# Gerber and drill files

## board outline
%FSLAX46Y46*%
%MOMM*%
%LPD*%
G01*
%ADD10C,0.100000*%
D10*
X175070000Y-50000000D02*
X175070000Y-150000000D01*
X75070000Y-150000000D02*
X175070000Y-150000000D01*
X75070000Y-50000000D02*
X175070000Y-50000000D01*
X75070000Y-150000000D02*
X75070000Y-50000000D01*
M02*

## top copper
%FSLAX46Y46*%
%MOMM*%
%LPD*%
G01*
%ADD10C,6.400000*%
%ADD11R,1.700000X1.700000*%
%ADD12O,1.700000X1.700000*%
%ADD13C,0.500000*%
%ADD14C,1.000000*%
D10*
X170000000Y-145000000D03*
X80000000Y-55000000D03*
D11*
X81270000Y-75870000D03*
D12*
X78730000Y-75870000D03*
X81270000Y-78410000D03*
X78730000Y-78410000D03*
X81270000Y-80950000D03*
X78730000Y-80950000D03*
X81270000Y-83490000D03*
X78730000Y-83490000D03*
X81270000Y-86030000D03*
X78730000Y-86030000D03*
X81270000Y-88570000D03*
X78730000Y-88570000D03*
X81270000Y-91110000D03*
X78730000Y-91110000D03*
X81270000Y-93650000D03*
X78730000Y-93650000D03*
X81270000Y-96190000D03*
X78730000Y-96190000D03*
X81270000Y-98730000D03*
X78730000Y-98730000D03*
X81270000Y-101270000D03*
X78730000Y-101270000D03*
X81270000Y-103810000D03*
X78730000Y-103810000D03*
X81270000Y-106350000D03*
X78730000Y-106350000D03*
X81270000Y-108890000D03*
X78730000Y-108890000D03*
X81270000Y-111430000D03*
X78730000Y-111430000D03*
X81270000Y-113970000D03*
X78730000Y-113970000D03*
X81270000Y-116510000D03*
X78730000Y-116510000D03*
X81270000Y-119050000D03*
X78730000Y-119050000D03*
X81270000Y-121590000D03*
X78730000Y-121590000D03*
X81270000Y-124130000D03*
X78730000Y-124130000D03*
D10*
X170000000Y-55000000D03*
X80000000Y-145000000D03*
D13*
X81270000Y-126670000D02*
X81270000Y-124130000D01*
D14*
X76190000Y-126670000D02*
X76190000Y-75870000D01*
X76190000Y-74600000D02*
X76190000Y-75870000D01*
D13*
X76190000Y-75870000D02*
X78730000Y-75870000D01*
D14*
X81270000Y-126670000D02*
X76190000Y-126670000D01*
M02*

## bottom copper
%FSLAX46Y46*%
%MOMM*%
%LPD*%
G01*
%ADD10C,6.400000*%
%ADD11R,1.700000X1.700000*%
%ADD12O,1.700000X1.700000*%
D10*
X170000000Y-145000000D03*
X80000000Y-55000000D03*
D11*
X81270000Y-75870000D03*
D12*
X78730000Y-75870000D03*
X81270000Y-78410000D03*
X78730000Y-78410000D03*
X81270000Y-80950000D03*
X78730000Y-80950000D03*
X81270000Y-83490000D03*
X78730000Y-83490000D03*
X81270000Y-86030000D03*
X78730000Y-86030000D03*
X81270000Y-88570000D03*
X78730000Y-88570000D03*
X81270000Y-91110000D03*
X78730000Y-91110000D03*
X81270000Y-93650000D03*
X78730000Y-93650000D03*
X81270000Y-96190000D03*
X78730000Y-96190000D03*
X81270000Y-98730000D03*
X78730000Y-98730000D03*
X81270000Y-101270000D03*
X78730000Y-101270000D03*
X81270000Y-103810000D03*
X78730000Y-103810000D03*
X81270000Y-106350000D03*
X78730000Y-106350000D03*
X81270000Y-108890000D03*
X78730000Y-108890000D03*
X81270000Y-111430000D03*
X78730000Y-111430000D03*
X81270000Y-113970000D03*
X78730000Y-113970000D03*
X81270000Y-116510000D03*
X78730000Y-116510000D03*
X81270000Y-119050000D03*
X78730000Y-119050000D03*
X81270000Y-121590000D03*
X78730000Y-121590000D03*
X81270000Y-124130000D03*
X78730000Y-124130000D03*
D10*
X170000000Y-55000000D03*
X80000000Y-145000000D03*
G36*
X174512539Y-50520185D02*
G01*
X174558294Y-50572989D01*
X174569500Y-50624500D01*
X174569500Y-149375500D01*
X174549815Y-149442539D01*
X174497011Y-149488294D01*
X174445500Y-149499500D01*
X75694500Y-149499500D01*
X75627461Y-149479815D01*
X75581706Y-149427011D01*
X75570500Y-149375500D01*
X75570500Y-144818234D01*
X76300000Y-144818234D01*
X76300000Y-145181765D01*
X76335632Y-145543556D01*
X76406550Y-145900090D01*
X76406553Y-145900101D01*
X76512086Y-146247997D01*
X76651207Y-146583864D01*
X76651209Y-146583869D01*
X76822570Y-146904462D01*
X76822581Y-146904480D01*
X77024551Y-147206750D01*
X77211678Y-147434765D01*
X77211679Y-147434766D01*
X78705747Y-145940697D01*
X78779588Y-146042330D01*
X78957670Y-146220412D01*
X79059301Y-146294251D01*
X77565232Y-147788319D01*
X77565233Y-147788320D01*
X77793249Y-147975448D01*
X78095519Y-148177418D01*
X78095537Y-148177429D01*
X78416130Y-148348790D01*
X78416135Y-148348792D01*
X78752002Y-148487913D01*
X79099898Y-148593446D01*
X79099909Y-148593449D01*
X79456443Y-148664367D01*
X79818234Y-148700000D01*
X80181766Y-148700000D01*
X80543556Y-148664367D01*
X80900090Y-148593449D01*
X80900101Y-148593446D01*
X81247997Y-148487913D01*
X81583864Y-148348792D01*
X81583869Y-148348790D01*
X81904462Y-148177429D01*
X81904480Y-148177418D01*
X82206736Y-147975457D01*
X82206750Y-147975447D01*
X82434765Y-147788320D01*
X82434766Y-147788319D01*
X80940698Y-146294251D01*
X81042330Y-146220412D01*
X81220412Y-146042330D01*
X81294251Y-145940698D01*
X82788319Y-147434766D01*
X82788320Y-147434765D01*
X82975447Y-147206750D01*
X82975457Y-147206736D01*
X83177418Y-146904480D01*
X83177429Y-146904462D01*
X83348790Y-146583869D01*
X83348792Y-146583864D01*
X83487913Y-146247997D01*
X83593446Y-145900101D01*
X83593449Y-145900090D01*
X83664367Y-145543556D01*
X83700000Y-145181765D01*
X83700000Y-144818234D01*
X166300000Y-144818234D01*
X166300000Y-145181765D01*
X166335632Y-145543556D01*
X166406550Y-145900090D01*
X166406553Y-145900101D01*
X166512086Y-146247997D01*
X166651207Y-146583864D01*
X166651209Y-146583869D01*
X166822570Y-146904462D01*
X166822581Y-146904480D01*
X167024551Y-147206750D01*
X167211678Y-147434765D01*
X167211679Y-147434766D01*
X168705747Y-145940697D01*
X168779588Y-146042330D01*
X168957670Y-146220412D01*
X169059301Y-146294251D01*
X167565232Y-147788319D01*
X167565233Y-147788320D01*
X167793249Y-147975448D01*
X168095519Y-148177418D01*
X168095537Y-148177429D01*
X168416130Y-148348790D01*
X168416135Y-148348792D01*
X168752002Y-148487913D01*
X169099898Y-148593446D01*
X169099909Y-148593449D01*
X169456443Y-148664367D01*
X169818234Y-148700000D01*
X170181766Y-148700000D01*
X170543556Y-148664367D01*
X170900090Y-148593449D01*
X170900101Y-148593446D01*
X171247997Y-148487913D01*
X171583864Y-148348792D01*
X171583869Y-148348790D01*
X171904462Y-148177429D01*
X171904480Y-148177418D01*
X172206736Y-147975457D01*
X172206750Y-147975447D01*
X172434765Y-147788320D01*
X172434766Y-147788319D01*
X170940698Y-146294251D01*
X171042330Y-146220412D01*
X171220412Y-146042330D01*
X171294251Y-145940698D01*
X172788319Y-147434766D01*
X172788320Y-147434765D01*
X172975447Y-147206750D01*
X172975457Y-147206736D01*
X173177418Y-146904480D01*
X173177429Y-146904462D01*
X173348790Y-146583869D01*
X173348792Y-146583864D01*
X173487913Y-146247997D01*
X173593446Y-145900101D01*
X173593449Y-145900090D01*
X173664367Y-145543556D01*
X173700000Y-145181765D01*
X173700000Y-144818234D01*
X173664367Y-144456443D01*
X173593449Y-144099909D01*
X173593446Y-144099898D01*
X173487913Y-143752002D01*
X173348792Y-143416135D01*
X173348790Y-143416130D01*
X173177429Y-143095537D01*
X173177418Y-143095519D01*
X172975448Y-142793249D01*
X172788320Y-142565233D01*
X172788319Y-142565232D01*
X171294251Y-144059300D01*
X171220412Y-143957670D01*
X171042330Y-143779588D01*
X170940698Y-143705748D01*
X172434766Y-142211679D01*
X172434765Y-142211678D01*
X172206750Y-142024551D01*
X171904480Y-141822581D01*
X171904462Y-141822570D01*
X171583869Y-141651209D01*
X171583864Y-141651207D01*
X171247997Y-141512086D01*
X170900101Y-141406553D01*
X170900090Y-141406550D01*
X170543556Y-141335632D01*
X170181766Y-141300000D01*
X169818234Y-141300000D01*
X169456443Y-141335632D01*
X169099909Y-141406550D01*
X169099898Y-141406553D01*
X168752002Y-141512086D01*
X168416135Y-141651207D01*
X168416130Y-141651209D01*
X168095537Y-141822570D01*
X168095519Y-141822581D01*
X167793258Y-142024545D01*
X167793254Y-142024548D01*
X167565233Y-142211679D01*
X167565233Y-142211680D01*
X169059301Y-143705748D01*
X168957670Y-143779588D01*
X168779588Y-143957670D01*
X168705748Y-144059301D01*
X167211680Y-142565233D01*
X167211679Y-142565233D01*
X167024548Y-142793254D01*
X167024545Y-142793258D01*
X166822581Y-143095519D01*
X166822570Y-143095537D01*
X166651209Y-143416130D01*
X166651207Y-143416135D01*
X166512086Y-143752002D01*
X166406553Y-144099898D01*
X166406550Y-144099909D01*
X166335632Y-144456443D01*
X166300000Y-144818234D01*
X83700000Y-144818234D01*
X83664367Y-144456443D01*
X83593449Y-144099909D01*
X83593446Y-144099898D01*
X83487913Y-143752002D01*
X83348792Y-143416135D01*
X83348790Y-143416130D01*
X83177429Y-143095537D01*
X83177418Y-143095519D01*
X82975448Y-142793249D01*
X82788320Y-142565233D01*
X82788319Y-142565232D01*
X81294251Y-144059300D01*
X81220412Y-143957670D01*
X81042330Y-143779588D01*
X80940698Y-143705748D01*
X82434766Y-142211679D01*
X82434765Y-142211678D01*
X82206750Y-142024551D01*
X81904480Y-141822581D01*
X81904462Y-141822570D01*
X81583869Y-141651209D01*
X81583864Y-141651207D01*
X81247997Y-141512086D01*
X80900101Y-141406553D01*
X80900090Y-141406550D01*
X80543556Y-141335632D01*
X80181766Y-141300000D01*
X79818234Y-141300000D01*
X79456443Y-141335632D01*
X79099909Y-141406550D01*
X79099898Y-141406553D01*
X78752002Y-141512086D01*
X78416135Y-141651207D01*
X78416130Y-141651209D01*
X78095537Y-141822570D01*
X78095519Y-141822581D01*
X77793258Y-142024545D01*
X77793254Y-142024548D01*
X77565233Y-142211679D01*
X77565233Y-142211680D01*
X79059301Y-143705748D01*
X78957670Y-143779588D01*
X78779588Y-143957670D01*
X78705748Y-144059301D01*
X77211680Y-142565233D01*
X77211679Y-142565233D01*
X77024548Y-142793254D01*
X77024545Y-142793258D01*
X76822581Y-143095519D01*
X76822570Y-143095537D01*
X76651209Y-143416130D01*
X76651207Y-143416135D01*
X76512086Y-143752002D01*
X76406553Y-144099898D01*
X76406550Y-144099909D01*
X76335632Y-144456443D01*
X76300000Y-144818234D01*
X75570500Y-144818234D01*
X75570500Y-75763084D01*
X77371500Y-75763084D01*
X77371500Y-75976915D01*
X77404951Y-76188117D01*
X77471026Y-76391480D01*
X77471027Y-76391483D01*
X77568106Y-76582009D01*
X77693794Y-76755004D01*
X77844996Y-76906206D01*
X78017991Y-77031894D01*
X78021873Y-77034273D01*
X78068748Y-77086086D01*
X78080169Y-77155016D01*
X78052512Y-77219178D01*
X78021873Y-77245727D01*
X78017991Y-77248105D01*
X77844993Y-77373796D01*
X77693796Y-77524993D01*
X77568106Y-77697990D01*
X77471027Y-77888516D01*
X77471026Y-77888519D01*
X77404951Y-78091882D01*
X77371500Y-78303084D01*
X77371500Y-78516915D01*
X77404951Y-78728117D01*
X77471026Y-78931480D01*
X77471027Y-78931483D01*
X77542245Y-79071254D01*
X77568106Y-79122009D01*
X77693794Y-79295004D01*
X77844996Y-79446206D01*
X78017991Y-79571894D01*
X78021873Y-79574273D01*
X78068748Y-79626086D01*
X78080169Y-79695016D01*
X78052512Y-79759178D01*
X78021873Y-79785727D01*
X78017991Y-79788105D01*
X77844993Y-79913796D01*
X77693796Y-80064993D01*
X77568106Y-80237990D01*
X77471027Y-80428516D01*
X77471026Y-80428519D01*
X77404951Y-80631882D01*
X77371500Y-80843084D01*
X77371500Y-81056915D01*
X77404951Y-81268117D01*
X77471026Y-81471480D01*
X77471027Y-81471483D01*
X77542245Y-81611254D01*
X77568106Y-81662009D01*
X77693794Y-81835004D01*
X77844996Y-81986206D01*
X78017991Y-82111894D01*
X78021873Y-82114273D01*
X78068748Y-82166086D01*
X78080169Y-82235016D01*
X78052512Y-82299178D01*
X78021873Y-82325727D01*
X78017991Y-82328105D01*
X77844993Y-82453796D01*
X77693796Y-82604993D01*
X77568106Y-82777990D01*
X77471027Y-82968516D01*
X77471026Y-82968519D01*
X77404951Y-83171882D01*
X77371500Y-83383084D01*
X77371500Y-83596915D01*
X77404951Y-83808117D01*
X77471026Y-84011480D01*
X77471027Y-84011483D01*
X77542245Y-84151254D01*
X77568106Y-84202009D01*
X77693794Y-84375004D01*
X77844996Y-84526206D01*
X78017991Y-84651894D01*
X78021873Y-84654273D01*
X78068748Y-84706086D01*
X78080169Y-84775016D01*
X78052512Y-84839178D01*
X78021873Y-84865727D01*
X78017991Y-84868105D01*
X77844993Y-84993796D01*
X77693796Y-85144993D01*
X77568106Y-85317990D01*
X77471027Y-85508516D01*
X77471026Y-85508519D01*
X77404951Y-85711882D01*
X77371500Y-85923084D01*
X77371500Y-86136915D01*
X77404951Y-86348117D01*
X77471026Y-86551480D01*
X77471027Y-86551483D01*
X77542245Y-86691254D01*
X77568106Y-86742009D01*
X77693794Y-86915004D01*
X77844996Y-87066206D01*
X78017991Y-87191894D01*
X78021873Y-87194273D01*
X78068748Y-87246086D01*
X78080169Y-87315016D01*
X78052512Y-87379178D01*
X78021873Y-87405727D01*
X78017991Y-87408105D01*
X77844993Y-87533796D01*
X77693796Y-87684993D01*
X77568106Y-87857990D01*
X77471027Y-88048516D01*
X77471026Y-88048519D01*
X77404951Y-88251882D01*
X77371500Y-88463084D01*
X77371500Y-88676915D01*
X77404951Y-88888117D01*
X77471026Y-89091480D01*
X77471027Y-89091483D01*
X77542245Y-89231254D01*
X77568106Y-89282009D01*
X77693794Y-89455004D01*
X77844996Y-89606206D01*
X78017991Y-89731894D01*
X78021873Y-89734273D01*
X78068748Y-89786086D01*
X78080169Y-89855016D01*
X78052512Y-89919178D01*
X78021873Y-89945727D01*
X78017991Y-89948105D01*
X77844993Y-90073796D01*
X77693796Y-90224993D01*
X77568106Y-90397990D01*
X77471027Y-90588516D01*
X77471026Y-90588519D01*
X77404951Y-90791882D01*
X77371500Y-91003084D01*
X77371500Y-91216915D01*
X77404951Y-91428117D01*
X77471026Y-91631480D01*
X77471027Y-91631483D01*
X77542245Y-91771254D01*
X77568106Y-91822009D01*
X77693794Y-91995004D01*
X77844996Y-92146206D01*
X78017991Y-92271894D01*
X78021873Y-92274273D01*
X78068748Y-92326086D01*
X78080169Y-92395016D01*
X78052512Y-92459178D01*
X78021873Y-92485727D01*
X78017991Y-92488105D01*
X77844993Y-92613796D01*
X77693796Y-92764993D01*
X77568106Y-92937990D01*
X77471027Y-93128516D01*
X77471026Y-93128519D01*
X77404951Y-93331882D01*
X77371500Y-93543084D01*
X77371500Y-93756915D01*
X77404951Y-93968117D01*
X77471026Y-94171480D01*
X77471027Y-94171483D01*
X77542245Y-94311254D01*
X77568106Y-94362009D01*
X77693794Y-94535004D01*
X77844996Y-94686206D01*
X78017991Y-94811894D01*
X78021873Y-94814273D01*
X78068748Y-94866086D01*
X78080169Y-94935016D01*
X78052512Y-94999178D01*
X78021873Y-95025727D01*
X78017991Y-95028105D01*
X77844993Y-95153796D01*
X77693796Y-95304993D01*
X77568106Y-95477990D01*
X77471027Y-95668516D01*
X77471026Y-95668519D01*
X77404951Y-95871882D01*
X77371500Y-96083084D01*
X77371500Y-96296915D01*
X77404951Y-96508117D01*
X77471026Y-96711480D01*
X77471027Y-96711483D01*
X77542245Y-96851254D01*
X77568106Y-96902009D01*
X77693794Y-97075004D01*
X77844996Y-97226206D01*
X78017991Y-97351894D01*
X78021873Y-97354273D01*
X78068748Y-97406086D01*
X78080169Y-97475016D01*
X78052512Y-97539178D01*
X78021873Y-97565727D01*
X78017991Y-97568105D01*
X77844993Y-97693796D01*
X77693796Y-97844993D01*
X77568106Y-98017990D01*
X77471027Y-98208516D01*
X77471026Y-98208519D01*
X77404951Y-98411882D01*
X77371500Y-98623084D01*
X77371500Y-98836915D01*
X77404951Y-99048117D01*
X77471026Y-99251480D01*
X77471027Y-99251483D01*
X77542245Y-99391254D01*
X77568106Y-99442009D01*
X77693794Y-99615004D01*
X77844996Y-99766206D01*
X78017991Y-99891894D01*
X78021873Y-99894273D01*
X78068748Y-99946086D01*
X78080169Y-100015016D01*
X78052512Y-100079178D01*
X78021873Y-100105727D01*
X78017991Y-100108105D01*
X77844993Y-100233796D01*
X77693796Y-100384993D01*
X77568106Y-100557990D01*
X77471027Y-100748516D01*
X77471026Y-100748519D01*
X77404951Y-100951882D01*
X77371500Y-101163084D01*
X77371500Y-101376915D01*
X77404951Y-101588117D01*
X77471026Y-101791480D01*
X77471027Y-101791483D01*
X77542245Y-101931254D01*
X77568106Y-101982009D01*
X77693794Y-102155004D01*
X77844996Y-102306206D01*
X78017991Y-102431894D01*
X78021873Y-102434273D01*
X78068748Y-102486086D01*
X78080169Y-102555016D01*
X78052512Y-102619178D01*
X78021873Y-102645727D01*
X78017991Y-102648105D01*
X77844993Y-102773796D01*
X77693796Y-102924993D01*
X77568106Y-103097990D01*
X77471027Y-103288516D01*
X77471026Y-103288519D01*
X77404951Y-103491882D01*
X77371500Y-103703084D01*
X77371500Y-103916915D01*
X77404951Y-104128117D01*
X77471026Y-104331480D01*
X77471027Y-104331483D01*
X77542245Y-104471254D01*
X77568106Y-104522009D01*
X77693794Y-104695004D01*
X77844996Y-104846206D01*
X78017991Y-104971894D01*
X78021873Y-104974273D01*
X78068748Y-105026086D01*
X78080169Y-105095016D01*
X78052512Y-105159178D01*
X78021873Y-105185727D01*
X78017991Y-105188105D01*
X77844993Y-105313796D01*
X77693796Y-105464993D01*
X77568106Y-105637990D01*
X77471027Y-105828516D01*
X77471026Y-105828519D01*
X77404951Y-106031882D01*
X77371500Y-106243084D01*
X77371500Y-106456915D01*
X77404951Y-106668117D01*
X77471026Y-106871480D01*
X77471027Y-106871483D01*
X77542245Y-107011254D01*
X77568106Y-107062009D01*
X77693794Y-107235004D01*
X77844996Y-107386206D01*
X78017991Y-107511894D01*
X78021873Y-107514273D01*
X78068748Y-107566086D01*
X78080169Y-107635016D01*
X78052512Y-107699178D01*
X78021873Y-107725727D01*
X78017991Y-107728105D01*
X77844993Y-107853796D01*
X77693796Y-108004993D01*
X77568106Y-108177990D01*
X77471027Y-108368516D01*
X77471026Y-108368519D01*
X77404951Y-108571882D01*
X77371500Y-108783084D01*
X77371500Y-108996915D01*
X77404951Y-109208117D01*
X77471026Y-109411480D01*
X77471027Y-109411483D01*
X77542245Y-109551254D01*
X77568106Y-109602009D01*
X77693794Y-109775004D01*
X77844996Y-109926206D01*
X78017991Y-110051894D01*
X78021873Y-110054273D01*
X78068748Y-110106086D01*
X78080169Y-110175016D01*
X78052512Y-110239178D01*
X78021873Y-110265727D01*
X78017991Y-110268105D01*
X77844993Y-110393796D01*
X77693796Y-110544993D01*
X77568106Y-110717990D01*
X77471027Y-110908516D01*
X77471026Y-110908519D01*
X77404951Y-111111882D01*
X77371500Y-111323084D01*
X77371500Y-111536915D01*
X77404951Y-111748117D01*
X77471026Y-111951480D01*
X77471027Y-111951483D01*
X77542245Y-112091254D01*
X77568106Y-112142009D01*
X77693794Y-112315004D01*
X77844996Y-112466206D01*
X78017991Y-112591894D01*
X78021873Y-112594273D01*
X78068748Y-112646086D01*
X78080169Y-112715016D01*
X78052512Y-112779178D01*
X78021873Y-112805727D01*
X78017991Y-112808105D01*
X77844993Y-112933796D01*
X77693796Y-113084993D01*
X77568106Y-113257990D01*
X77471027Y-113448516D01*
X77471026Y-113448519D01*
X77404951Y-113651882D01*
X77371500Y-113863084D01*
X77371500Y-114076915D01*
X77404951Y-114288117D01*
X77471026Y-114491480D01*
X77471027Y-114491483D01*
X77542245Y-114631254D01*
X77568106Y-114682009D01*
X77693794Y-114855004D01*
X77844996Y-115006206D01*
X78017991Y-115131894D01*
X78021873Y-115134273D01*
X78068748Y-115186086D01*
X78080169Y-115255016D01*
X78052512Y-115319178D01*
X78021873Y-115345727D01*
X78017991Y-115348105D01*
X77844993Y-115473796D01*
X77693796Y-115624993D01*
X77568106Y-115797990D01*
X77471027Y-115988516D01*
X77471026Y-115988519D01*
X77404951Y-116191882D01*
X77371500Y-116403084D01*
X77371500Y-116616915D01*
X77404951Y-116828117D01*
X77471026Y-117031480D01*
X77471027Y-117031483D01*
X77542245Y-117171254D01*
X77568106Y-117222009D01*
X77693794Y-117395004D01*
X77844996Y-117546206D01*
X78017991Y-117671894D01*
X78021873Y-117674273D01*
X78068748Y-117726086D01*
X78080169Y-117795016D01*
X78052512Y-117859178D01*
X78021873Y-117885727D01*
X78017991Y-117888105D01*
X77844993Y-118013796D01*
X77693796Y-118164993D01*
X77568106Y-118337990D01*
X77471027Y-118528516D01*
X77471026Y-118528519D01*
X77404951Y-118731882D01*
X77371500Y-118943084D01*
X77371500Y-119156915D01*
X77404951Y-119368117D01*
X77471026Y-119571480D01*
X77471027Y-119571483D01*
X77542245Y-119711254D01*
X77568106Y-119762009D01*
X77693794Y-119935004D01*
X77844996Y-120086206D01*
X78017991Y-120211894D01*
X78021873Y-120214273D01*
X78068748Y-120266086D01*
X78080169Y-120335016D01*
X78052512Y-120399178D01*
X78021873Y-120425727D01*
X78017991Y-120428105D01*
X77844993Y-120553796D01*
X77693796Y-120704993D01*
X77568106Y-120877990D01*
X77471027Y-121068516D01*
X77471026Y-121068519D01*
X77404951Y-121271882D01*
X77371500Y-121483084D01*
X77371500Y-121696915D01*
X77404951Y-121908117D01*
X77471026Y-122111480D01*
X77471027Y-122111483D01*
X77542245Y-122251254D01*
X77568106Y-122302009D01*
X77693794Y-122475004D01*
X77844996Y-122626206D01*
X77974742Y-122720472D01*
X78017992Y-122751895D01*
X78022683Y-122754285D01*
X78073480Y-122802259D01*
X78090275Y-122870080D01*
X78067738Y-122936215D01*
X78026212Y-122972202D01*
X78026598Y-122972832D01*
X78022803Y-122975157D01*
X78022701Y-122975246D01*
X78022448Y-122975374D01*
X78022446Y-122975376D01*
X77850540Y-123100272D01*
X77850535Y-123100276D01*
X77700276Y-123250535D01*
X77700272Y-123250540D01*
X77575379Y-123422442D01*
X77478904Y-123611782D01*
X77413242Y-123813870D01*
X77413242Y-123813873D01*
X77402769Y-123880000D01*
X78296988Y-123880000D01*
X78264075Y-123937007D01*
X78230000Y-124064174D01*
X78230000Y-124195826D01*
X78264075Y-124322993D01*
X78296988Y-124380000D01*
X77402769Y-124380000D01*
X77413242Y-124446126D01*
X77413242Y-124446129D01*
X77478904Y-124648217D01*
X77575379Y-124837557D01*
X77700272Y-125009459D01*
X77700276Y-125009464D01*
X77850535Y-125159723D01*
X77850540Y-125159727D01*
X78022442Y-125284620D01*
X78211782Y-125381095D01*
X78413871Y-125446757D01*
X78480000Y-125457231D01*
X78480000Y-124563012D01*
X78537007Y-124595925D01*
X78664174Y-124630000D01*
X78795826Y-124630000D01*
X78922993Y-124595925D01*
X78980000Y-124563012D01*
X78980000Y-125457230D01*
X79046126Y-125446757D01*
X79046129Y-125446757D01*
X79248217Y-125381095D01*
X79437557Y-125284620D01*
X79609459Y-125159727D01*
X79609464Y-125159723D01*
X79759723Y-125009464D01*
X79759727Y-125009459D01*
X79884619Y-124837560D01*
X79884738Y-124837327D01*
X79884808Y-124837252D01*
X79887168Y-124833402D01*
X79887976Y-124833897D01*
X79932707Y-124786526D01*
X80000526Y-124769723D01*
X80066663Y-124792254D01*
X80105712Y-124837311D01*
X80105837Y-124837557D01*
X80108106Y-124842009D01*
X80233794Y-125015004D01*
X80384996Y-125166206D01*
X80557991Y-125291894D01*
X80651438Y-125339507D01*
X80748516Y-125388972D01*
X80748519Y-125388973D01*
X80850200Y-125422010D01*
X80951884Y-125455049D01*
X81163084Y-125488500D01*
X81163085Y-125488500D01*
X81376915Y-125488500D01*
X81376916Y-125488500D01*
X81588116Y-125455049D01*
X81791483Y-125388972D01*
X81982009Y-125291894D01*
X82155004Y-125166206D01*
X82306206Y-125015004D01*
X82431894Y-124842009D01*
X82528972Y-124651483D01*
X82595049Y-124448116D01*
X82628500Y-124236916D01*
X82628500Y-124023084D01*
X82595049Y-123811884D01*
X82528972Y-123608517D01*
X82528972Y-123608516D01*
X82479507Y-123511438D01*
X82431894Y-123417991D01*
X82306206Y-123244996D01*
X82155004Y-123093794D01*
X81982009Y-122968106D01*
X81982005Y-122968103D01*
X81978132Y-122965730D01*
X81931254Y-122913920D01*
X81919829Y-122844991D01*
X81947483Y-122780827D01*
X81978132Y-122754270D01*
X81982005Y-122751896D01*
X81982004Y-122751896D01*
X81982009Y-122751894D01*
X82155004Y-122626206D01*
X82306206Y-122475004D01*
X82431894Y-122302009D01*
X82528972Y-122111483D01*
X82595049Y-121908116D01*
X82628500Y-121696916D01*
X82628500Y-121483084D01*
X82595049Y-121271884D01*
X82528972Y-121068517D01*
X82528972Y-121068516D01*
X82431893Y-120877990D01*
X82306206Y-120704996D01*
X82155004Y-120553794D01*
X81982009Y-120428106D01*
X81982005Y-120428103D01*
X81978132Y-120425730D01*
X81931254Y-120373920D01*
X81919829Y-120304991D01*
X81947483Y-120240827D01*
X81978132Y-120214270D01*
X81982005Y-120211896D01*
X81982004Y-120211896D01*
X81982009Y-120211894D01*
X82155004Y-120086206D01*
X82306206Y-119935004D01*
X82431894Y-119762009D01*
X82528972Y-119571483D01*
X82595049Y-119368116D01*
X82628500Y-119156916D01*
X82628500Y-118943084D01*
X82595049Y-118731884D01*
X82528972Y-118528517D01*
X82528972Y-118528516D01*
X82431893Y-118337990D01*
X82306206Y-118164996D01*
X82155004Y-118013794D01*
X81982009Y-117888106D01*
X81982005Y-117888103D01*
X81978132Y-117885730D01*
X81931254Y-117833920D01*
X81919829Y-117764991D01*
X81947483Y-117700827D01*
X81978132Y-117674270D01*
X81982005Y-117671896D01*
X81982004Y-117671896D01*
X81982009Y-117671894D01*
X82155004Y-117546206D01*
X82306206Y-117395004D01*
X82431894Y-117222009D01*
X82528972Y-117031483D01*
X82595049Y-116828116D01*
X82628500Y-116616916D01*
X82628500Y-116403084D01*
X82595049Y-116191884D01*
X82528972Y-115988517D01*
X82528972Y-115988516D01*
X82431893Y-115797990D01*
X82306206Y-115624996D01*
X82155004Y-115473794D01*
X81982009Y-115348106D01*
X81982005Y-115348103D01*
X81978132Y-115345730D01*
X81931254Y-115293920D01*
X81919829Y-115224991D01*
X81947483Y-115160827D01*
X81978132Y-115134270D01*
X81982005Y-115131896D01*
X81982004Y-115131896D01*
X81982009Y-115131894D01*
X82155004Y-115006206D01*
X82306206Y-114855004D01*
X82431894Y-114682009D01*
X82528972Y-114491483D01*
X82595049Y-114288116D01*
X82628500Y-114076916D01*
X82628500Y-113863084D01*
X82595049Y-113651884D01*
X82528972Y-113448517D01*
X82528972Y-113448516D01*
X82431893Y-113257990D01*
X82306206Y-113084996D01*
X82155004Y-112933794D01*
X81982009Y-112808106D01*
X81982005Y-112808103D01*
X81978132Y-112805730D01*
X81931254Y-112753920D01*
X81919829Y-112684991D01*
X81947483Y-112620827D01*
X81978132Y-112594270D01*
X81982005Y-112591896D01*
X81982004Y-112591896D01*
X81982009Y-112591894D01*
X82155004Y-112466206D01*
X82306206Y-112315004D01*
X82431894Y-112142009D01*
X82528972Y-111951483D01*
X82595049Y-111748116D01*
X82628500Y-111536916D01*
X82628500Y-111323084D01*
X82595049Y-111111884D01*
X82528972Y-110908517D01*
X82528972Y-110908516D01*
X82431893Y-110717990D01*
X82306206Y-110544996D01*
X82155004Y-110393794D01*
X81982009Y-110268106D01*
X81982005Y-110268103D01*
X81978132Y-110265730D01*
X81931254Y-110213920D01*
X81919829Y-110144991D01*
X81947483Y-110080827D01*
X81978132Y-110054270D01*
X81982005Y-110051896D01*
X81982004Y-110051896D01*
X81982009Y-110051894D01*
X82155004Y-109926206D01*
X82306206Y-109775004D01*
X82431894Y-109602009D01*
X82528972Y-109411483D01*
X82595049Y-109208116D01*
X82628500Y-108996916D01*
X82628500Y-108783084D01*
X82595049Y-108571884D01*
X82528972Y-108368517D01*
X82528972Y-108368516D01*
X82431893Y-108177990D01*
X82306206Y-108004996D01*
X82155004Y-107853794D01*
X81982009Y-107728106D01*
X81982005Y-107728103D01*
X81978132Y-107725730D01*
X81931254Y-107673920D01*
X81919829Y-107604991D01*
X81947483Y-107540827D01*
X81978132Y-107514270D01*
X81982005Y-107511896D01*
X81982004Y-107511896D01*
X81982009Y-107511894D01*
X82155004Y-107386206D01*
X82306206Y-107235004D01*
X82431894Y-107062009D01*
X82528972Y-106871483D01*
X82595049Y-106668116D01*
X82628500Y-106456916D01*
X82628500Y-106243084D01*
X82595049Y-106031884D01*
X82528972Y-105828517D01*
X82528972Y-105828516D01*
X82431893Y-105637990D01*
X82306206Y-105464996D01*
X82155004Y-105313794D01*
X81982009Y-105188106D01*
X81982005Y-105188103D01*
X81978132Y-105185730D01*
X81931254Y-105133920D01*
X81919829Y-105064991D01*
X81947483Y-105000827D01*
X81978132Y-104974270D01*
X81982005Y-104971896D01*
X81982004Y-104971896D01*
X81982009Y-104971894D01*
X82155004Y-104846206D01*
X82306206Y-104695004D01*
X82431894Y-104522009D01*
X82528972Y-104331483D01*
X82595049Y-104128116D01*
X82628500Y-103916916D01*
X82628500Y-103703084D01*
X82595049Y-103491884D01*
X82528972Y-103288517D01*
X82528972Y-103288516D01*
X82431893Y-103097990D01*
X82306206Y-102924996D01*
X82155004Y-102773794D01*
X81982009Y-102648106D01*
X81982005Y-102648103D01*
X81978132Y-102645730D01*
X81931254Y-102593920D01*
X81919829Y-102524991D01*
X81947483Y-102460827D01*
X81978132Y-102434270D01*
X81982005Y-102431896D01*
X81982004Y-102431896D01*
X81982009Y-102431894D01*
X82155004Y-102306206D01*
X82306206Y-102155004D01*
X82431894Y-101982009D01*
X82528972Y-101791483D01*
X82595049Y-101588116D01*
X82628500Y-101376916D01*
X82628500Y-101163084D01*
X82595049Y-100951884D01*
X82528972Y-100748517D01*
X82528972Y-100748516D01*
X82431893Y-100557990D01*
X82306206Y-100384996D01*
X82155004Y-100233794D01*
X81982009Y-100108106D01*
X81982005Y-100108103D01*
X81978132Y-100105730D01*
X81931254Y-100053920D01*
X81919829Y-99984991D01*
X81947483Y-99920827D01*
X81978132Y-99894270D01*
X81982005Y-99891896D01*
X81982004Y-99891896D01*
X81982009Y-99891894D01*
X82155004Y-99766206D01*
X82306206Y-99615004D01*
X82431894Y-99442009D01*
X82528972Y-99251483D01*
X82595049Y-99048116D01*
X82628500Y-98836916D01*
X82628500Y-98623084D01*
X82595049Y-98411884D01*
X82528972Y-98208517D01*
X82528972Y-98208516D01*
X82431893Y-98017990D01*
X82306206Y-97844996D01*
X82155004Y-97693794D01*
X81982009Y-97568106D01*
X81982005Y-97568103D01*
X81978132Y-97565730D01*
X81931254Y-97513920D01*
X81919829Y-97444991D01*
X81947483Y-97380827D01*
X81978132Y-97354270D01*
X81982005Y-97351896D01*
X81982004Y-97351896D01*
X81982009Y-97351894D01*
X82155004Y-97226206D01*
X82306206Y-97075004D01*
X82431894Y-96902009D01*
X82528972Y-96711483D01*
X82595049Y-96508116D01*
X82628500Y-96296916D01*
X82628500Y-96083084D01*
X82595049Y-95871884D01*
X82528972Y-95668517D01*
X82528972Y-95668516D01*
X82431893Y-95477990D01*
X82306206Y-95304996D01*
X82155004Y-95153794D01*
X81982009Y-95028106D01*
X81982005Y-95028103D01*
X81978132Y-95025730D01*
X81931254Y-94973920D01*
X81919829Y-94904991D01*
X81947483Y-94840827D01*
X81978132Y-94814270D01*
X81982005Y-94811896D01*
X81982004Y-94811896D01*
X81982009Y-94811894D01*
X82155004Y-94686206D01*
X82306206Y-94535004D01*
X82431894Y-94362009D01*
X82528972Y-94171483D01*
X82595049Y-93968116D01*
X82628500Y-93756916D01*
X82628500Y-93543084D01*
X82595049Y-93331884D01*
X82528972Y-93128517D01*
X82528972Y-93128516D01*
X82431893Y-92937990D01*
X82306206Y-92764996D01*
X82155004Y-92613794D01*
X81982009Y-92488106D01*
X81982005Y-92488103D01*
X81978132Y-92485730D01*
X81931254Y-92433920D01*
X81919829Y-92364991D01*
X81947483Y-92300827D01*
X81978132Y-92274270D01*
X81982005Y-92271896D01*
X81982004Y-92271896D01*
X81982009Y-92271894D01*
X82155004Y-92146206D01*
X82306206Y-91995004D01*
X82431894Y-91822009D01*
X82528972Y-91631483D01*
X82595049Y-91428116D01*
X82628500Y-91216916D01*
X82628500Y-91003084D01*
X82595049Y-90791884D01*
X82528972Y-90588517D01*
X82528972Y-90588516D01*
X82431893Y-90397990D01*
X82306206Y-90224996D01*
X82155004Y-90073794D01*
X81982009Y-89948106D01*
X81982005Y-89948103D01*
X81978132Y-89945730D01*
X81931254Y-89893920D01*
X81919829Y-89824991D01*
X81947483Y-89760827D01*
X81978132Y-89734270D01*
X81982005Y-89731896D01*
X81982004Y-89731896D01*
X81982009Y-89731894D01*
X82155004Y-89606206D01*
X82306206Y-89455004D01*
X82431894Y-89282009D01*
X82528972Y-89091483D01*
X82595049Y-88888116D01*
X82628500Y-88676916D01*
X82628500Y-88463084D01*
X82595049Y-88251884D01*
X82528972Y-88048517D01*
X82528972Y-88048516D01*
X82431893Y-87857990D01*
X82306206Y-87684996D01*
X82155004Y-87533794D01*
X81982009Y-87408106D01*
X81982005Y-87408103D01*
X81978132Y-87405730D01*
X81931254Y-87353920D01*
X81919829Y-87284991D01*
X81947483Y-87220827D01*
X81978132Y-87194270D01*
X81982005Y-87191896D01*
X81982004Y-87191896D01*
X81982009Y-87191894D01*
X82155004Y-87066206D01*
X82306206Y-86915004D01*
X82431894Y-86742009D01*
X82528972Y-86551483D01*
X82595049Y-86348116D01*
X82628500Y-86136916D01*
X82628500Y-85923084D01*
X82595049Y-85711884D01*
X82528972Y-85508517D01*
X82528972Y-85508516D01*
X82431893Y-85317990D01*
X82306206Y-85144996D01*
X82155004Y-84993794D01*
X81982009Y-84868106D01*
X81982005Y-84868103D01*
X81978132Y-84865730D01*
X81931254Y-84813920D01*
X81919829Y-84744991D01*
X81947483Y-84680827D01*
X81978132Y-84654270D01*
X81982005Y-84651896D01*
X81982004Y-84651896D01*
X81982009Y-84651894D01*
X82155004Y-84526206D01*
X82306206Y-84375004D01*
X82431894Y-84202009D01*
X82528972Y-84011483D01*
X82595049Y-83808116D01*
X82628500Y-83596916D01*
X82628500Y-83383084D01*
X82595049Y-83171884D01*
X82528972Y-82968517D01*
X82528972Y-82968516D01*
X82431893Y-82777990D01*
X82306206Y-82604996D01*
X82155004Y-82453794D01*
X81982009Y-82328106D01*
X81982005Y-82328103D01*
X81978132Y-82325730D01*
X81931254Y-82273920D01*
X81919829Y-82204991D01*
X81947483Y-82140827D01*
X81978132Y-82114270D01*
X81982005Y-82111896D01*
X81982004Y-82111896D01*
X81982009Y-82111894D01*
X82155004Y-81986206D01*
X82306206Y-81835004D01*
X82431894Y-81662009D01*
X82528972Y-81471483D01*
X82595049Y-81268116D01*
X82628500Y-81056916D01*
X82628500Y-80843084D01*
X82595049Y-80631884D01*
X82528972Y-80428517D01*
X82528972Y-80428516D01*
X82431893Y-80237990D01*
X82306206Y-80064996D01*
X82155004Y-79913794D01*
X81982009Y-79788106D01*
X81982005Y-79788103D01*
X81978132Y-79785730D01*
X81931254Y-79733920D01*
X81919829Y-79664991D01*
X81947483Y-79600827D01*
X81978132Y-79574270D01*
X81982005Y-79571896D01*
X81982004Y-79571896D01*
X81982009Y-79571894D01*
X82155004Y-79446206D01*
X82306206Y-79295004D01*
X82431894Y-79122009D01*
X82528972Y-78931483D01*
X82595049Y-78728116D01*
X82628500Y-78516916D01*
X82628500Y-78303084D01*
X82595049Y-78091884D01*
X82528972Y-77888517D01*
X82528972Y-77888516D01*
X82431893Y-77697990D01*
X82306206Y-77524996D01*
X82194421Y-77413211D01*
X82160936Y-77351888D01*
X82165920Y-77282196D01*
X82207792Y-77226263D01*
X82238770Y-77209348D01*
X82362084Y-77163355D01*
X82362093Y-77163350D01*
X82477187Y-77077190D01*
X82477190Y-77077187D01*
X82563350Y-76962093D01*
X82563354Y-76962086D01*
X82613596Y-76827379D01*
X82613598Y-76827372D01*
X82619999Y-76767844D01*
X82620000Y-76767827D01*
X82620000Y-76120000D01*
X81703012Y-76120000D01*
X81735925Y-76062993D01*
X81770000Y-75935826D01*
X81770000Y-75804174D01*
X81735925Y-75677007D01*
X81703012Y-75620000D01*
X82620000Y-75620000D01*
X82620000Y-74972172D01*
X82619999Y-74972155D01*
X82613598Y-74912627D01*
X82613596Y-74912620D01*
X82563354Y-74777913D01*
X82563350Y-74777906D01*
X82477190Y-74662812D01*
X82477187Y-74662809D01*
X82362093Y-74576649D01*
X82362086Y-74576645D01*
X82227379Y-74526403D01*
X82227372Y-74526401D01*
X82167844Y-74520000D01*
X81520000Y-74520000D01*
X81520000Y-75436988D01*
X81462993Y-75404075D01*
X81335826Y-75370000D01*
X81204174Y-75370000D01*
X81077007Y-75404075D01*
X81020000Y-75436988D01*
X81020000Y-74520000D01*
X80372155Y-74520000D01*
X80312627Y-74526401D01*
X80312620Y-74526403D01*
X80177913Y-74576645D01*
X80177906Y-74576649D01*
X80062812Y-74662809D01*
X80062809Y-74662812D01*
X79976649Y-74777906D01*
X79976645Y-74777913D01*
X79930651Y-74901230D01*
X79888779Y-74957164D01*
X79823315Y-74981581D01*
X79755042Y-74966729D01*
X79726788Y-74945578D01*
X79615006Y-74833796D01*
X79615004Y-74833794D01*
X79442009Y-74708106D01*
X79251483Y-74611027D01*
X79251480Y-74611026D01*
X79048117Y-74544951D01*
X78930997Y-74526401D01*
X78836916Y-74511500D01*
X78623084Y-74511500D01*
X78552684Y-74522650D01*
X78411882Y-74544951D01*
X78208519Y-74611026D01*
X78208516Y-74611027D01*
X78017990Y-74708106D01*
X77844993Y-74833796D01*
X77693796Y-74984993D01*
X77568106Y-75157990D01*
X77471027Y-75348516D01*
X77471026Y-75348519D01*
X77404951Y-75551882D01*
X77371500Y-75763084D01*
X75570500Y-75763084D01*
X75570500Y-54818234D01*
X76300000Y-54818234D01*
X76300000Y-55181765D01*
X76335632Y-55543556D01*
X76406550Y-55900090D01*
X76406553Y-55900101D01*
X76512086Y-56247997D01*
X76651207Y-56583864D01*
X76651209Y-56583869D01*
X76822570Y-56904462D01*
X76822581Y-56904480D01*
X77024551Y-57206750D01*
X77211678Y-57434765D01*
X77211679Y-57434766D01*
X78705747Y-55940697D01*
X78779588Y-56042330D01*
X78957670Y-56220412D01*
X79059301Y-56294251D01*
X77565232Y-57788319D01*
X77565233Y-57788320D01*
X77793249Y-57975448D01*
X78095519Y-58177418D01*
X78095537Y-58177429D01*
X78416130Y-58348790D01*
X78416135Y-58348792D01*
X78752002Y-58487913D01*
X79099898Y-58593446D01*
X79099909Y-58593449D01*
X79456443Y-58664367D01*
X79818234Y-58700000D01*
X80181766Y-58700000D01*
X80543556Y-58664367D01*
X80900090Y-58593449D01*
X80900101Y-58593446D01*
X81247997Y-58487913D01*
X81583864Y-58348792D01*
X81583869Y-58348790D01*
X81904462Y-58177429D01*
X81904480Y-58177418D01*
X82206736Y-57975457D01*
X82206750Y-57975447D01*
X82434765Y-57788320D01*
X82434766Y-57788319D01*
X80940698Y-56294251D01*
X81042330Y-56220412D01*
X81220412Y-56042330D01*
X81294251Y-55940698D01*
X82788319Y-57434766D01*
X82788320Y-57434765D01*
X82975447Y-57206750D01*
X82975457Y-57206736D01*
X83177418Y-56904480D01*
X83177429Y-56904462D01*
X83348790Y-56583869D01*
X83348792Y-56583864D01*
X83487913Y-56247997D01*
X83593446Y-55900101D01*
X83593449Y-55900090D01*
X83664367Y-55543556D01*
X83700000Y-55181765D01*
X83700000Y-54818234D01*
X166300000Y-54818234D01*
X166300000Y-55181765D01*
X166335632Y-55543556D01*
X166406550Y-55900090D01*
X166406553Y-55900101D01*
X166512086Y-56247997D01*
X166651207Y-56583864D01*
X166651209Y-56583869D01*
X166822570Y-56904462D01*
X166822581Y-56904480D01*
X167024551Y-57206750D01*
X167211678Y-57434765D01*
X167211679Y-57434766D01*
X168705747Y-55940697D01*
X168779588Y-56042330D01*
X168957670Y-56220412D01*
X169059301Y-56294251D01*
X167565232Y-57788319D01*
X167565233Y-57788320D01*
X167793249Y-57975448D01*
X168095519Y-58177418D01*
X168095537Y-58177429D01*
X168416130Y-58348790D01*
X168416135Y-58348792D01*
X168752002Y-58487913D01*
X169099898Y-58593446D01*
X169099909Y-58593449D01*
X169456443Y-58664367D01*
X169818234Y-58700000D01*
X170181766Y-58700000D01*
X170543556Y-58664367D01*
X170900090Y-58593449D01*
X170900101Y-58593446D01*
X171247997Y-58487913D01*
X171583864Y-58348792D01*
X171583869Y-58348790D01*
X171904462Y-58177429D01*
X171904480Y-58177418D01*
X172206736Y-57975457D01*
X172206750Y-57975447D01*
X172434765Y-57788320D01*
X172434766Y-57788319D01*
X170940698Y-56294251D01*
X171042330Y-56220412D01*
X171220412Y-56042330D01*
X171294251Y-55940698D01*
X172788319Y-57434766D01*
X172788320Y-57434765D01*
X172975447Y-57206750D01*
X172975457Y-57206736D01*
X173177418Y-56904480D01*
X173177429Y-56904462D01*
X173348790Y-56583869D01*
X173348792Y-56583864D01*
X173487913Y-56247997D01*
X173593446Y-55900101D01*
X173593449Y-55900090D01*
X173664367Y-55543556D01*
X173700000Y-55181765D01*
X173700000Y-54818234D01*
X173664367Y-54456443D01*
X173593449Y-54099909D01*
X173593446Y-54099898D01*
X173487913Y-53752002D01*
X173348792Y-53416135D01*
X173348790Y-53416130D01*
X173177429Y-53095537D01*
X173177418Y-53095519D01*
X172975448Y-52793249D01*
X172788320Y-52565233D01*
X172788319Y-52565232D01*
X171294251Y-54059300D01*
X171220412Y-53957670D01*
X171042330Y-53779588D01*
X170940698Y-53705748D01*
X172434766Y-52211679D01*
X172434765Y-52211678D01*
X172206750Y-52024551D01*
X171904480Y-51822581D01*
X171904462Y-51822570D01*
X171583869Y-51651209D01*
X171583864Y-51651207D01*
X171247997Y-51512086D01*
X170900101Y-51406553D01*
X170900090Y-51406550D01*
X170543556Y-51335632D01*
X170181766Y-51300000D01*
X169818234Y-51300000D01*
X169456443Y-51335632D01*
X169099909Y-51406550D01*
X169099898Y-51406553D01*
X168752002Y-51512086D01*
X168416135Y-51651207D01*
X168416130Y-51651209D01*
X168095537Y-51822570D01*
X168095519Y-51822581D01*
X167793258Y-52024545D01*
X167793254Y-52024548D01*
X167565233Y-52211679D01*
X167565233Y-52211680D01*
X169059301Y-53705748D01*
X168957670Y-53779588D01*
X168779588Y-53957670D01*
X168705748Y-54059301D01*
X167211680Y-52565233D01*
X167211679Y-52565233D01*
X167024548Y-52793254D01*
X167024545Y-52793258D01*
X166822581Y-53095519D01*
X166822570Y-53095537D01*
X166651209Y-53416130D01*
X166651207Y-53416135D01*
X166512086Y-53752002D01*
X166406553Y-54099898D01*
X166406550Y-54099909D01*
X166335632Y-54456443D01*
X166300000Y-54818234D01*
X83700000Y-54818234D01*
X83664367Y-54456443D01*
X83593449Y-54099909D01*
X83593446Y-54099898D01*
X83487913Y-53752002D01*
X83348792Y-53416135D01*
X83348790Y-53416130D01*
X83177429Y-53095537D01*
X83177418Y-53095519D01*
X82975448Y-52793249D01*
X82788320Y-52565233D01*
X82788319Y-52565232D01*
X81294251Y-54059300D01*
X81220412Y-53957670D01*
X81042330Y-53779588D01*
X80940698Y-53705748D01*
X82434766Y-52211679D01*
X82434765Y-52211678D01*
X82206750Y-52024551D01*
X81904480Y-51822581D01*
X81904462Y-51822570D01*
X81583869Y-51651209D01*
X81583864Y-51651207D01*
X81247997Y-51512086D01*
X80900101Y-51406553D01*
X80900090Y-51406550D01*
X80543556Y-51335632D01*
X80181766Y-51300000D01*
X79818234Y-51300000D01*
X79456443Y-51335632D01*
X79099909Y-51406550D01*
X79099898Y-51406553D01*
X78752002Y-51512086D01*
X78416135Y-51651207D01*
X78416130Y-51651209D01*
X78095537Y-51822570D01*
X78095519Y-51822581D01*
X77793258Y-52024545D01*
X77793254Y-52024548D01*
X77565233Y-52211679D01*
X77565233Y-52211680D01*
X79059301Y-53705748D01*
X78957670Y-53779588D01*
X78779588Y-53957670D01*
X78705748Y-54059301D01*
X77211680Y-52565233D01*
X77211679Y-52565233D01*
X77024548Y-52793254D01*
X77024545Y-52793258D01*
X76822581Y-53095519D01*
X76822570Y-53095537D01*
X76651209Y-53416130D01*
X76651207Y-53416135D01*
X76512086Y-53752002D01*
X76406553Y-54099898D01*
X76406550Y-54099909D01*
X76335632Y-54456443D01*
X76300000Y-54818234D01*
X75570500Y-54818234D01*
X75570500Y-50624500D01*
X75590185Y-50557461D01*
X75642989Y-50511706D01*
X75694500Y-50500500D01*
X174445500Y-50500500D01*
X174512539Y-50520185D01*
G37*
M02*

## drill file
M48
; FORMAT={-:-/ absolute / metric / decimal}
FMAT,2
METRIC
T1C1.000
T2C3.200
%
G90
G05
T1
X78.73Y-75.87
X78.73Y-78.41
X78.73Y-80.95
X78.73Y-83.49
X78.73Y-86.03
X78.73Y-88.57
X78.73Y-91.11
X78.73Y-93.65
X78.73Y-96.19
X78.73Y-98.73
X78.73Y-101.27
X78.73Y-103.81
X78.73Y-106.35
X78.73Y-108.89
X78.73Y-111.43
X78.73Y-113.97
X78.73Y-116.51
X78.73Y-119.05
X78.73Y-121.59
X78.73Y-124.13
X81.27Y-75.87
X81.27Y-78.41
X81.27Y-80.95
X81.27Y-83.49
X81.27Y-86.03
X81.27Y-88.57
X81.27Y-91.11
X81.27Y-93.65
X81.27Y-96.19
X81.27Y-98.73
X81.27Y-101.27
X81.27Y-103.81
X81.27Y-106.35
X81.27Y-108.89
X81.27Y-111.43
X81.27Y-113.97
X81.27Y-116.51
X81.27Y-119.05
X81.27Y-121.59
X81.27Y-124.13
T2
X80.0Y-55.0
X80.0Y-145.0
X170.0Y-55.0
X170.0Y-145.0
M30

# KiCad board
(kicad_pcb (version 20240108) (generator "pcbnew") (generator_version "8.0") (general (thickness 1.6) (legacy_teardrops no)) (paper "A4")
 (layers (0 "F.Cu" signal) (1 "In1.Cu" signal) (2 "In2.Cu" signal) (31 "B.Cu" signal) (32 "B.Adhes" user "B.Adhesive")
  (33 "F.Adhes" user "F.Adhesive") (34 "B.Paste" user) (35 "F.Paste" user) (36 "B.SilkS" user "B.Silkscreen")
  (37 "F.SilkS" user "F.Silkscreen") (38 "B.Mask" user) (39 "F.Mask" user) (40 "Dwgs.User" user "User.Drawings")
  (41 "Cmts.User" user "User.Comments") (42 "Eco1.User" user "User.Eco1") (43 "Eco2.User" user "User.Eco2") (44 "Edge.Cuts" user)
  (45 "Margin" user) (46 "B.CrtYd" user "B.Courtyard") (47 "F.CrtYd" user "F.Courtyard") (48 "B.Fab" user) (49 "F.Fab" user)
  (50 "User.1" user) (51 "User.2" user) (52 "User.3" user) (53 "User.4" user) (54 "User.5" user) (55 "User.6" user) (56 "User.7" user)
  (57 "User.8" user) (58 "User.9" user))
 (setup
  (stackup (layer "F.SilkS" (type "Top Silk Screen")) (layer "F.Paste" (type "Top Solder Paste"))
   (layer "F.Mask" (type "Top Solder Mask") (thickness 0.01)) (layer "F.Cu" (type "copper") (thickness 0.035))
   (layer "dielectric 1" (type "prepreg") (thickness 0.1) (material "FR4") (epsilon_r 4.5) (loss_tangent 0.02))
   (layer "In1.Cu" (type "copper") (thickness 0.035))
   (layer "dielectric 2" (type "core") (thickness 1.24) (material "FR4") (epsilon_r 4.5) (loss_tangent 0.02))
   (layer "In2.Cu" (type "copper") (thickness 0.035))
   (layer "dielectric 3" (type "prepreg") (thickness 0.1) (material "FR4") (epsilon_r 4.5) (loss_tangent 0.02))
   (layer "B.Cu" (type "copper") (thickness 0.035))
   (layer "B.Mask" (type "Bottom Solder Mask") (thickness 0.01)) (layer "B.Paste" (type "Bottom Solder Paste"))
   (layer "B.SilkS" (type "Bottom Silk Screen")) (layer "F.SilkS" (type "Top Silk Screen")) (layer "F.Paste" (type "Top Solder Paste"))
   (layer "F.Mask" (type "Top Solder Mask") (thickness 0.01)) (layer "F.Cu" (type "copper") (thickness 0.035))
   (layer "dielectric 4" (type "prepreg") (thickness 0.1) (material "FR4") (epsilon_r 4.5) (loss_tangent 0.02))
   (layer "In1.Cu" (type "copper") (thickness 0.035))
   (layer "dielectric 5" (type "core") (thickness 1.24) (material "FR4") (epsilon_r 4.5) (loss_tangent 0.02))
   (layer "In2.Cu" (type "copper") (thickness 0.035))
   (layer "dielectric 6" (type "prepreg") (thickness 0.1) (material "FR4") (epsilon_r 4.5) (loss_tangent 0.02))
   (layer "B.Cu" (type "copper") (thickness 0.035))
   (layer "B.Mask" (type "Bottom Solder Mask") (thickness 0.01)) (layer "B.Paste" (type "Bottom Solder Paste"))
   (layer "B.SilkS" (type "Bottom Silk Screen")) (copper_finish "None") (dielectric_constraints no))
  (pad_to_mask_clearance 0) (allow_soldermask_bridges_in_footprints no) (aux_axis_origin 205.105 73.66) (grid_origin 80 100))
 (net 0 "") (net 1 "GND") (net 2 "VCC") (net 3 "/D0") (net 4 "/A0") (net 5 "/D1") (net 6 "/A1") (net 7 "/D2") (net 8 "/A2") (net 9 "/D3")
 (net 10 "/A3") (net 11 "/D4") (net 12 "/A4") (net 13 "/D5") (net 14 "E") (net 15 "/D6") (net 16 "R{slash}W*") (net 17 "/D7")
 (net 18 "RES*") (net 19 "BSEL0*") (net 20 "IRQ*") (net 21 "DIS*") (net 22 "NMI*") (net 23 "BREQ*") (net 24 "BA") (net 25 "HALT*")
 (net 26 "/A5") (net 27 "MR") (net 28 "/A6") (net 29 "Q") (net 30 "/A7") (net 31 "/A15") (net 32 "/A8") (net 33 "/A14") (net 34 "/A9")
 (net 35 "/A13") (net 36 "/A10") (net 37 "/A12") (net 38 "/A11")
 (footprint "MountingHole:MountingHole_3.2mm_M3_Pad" (layer "F.Cu") (at 170 145)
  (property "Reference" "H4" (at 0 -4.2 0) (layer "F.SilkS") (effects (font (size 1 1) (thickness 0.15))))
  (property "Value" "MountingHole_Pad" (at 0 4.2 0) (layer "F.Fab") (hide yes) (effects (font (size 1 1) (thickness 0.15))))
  (pad "1" thru_hole circle (at 0 0) (size 6.4 6.4) (drill 3.2) (layers "*.Cu" "*.Mask") (remove_unused_layers no) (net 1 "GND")))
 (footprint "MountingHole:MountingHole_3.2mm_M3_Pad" (layer "F.Cu") (at 80 55)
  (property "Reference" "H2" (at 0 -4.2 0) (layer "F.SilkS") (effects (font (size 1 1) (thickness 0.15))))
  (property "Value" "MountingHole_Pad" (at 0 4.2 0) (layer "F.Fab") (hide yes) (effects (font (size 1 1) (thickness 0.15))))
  (pad "1" thru_hole circle (at 0 0) (size 6.4 6.4) (drill 3.2) (layers "*.Cu" "*.Mask") (remove_unused_layers no) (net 1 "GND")))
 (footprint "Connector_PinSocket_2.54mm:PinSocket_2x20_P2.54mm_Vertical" (layer "F.Cu") (at 81.27 75.87)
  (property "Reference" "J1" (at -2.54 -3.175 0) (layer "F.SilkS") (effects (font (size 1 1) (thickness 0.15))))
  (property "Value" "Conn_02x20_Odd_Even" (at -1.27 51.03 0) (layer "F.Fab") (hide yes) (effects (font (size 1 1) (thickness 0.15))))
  (pad "1" thru_hole rect (at 0 0) (size 1.7 1.7) (drill 1) (layers "*.Cu" "*.Mask") (remove_unused_layers no) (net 1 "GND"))
  (pad "2" thru_hole oval (at -2.54 0) (size 1.7 1.7) (drill 1) (layers "*.Cu" "*.Mask") (remove_unused_layers no) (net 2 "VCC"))
  (pad "3" thru_hole oval (at 0 2.54) (size 1.7 1.7) (drill 1) (layers "*.Cu" "*.Mask") (remove_unused_layers no) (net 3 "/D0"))
  (pad "4" thru_hole oval (at -2.54 2.54) (size 1.7 1.7) (drill 1) (layers "*.Cu" "*.Mask") (remove_unused_layers no) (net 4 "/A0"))
  (pad "5" thru_hole oval (at 0 5.08) (size 1.7 1.7) (drill 1) (layers "*.Cu" "*.Mask") (remove_unused_layers no) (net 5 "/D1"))
  (pad "6" thru_hole oval (at -2.54 5.08) (size 1.7 1.7) (drill 1) (layers "*.Cu" "*.Mask") (remove_unused_layers no) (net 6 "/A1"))
  (pad "7" thru_hole oval (at 0 7.62) (size 1.7 1.7) (drill 1) (layers "*.Cu" "*.Mask") (remove_unused_layers no) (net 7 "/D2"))
  (pad "8" thru_hole oval (at -2.54 7.62) (size 1.7 1.7) (drill 1) (layers "*.Cu" "*.Mask") (remove_unused_layers no) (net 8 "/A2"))
  (pad "9" thru_hole oval (at 0 10.16) (size 1.7 1.7) (drill 1) (layers "*.Cu" "*.Mask") (remove_unused_layers no) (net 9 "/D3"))
  (pad "10" thru_hole oval (at -2.54 10.16) (size 1.7 1.7) (drill 1) (layers "*.Cu" "*.Mask") (remove_unused_layers no) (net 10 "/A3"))
  (pad "11" thru_hole oval (at 0 12.7) (size 1.7 1.7) (drill 1) (layers "*.Cu" "*.Mask") (remove_unused_layers no) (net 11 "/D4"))
  (pad "12" thru_hole oval (at -2.54 12.7) (size 1.7 1.7) (drill 1) (layers "*.Cu" "*.Mask") (remove_unused_layers no) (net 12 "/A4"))
  (pad "13" thru_hole oval (at 0 15.24) (size 1.7 1.7) (drill 1) (layers "*.Cu" "*.Mask") (remove_unused_layers no) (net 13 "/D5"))
  (pad "14" thru_hole oval (at -2.54 15.24) (size 1.7 1.7) (drill 1) (layers "*.Cu" "*.Mask") (remove_unused_layers no) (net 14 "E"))
  (pad "15" thru_hole oval (at 0 17.78) (size 1.7 1.7) (drill 1) (layers "*.Cu" "*.Mask") (remove_unused_layers no) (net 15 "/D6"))
  (pad "16" thru_hole oval (at -2.54 17.78) (size 1.7 1.7) (drill 1) (layers "*.Cu" "*.Mask") (remove_unused_layers no)
   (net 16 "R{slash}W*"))
  (pad "17" thru_hole oval (at 0 20.32) (size 1.7 1.7) (drill 1) (layers "*.Cu" "*.Mask") (remove_unused_layers no) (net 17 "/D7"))
  (pad "18" thru_hole oval (at -2.54 20.32) (size 1.7 1.7) (drill 1) (layers "*.Cu" "*.Mask") (remove_unused_layers no) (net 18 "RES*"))
  (pad "19" thru_hole oval (at 0 22.86) (size 1.7 1.7) (drill 1) (layers "*.Cu" "*.Mask") (remove_unused_layers no) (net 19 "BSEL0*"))
  (pad "20" thru_hole oval (at -2.54 22.86) (size 1.7 1.7) (drill 1) (layers "*.Cu" "*.Mask") (remove_unused_layers no) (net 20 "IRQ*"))
  (pad "21" thru_hole oval (at 0 25.4) (size 1.7 1.7) (drill 1) (layers "*.Cu" "*.Mask") (remove_unused_layers no) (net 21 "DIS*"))
  (pad "22" thru_hole oval (at -2.54 25.4) (size 1.7 1.7) (drill 1) (layers "*.Cu" "*.Mask") (remove_unused_layers no) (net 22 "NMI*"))
  (pad "23" thru_hole oval (at 0 27.94) (size 1.7 1.7) (drill 1) (layers "*.Cu" "*.Mask") (remove_unused_layers no) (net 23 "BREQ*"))
  (pad "24" thru_hole oval (at -2.54 27.94) (size 1.7 1.7) (drill 1) (layers "*.Cu" "*.Mask") (remove_unused_layers no) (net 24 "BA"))
  (pad "25" thru_hole oval (at 0 30.48) (size 1.7 1.7) (drill 1) (layers "*.Cu" "*.Mask") (remove_unused_layers no) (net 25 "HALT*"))
  (pad "26" thru_hole oval (at -2.54 30.48) (size 1.7 1.7) (drill 1) (layers "*.Cu" "*.Mask") (remove_unused_layers no) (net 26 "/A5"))
  (pad "27" thru_hole oval (at 0 33.02) (size 1.7 1.7) (drill 1) (layers "*.Cu" "*.Mask") (remove_unused_layers no) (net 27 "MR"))
  (pad "28" thru_hole oval (at -2.54 33.02) (size 1.7 1.7) (drill 1) (layers "*.Cu" "*.Mask") (remove_unused_layers no) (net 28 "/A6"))
  (pad "29" thru_hole oval (at 0 35.56) (size 1.7 1.7) (drill 1) (layers "*.Cu" "*.Mask") (remove_unused_layers no) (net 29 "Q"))
  (pad "30" thru_hole oval (at -2.54 35.56) (size 1.7 1.7) (drill 1) (layers "*.Cu" "*.Mask") (remove_unused_layers no) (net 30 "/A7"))
  (pad "31" thru_hole oval (at 0 38.1) (size 1.7 1.7) (drill 1) (layers "*.Cu" "*.Mask") (remove_unused_layers no) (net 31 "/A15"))
  (pad "32" thru_hole oval (at -2.54 38.1) (size 1.7 1.7) (drill 1) (layers "*.Cu" "*.Mask") (remove_unused_layers no) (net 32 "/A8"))
  (pad "33" thru_hole oval (at 0 40.64) (size 1.7 1.7) (drill 1) (layers "*.Cu" "*.Mask") (remove_unused_layers no) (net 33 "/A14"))
  (pad "34" thru_hole oval (at -2.54 40.64) (size 1.7 1.7) (drill 1) (layers "*.Cu" "*.Mask") (remove_unused_layers no) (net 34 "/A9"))
  (pad "35" thru_hole oval (at 0 43.18) (size 1.7 1.7) (drill 1) (layers "*.Cu" "*.Mask") (remove_unused_layers no) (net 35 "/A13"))
  (pad "36" thru_hole oval (at -2.54 43.18) (size 1.7 1.7) (drill 1) (layers "*.Cu" "*.Mask") (remove_unused_layers no) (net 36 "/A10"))
  (pad "37" thru_hole oval (at 0 45.72) (size 1.7 1.7) (drill 1) (layers "*.Cu" "*.Mask") (remove_unused_layers no) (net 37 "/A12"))
  (pad "38" thru_hole oval (at -2.54 45.72) (size 1.7 1.7) (drill 1) (layers "*.Cu" "*.Mask") (remove_unused_layers no) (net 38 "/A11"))
  (pad "39" thru_hole oval (at 0 48.26) (size 1.7 1.7) (drill 1) (layers "*.Cu" "*.Mask") (remove_unused_layers no) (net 2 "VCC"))
  (pad "40" thru_hole oval (at -2.54 48.26) (size 1.7 1.7) (drill 1) (layers "*.Cu" "*.Mask") (remove_unused_layers no) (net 1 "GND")))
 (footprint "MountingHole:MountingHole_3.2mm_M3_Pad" (layer "F.Cu") (at 170 55)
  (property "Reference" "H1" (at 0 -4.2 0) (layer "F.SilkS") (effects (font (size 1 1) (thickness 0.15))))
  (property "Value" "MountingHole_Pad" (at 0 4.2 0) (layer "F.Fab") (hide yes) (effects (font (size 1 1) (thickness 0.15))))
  (pad "1" thru_hole circle (at 0 0) (size 6.4 6.4) (drill 3.2) (layers "*.Cu" "*.Mask") (remove_unused_layers no) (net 1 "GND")))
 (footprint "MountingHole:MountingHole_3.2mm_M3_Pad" (layer "F.Cu") (at 80 145)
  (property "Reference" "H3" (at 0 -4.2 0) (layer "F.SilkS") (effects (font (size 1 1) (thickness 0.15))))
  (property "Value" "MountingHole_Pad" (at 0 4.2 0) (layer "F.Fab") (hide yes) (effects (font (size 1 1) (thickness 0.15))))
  (pad "1" thru_hole circle (at 0 0) (size 6.4 6.4) (drill 3.2) (layers "*.Cu" "*.Mask") (remove_unused_layers no) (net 1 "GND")))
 (gr_line (start 175.07 50) (end 175.07 150) (stroke (width 0.1) (type solid)) (layer "Edge.Cuts"))
 (gr_line (start 75.07 150) (end 175.07 150) (stroke (width 0.1) (type solid)) (layer "Edge.Cuts"))
 (gr_line (start 75.07 50) (end 175.07 50) (stroke (width 0.1) (type solid)) (layer "Edge.Cuts"))
 (gr_line (start 75.07 150) (end 75.07 50) (stroke (width 0.1) (type solid)) (layer "Edge.Cuts"))
 (segment (start 81.27 126.67) (end 81.27 124.13) (width 0.5) (layer "F.Cu") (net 2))
 (segment (start 76.19 126.67) (end 76.19 75.87) (width 1) (layer "F.Cu") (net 2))
 (segment (start 76.19 74.6) (end 76.19 75.87) (width 1) (layer "F.Cu") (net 2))
 (segment (start 76.19 75.87) (end 78.73 75.87) (width 0.5) (layer "F.Cu") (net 2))
 (segment (start 81.27 126.67) (end 76.19 126.67) (width 1) (layer "F.Cu") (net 2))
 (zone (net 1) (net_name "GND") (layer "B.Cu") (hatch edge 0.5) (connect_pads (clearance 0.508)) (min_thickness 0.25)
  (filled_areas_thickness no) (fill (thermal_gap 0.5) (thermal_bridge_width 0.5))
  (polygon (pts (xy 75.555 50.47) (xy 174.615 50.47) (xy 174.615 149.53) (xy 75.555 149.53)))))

